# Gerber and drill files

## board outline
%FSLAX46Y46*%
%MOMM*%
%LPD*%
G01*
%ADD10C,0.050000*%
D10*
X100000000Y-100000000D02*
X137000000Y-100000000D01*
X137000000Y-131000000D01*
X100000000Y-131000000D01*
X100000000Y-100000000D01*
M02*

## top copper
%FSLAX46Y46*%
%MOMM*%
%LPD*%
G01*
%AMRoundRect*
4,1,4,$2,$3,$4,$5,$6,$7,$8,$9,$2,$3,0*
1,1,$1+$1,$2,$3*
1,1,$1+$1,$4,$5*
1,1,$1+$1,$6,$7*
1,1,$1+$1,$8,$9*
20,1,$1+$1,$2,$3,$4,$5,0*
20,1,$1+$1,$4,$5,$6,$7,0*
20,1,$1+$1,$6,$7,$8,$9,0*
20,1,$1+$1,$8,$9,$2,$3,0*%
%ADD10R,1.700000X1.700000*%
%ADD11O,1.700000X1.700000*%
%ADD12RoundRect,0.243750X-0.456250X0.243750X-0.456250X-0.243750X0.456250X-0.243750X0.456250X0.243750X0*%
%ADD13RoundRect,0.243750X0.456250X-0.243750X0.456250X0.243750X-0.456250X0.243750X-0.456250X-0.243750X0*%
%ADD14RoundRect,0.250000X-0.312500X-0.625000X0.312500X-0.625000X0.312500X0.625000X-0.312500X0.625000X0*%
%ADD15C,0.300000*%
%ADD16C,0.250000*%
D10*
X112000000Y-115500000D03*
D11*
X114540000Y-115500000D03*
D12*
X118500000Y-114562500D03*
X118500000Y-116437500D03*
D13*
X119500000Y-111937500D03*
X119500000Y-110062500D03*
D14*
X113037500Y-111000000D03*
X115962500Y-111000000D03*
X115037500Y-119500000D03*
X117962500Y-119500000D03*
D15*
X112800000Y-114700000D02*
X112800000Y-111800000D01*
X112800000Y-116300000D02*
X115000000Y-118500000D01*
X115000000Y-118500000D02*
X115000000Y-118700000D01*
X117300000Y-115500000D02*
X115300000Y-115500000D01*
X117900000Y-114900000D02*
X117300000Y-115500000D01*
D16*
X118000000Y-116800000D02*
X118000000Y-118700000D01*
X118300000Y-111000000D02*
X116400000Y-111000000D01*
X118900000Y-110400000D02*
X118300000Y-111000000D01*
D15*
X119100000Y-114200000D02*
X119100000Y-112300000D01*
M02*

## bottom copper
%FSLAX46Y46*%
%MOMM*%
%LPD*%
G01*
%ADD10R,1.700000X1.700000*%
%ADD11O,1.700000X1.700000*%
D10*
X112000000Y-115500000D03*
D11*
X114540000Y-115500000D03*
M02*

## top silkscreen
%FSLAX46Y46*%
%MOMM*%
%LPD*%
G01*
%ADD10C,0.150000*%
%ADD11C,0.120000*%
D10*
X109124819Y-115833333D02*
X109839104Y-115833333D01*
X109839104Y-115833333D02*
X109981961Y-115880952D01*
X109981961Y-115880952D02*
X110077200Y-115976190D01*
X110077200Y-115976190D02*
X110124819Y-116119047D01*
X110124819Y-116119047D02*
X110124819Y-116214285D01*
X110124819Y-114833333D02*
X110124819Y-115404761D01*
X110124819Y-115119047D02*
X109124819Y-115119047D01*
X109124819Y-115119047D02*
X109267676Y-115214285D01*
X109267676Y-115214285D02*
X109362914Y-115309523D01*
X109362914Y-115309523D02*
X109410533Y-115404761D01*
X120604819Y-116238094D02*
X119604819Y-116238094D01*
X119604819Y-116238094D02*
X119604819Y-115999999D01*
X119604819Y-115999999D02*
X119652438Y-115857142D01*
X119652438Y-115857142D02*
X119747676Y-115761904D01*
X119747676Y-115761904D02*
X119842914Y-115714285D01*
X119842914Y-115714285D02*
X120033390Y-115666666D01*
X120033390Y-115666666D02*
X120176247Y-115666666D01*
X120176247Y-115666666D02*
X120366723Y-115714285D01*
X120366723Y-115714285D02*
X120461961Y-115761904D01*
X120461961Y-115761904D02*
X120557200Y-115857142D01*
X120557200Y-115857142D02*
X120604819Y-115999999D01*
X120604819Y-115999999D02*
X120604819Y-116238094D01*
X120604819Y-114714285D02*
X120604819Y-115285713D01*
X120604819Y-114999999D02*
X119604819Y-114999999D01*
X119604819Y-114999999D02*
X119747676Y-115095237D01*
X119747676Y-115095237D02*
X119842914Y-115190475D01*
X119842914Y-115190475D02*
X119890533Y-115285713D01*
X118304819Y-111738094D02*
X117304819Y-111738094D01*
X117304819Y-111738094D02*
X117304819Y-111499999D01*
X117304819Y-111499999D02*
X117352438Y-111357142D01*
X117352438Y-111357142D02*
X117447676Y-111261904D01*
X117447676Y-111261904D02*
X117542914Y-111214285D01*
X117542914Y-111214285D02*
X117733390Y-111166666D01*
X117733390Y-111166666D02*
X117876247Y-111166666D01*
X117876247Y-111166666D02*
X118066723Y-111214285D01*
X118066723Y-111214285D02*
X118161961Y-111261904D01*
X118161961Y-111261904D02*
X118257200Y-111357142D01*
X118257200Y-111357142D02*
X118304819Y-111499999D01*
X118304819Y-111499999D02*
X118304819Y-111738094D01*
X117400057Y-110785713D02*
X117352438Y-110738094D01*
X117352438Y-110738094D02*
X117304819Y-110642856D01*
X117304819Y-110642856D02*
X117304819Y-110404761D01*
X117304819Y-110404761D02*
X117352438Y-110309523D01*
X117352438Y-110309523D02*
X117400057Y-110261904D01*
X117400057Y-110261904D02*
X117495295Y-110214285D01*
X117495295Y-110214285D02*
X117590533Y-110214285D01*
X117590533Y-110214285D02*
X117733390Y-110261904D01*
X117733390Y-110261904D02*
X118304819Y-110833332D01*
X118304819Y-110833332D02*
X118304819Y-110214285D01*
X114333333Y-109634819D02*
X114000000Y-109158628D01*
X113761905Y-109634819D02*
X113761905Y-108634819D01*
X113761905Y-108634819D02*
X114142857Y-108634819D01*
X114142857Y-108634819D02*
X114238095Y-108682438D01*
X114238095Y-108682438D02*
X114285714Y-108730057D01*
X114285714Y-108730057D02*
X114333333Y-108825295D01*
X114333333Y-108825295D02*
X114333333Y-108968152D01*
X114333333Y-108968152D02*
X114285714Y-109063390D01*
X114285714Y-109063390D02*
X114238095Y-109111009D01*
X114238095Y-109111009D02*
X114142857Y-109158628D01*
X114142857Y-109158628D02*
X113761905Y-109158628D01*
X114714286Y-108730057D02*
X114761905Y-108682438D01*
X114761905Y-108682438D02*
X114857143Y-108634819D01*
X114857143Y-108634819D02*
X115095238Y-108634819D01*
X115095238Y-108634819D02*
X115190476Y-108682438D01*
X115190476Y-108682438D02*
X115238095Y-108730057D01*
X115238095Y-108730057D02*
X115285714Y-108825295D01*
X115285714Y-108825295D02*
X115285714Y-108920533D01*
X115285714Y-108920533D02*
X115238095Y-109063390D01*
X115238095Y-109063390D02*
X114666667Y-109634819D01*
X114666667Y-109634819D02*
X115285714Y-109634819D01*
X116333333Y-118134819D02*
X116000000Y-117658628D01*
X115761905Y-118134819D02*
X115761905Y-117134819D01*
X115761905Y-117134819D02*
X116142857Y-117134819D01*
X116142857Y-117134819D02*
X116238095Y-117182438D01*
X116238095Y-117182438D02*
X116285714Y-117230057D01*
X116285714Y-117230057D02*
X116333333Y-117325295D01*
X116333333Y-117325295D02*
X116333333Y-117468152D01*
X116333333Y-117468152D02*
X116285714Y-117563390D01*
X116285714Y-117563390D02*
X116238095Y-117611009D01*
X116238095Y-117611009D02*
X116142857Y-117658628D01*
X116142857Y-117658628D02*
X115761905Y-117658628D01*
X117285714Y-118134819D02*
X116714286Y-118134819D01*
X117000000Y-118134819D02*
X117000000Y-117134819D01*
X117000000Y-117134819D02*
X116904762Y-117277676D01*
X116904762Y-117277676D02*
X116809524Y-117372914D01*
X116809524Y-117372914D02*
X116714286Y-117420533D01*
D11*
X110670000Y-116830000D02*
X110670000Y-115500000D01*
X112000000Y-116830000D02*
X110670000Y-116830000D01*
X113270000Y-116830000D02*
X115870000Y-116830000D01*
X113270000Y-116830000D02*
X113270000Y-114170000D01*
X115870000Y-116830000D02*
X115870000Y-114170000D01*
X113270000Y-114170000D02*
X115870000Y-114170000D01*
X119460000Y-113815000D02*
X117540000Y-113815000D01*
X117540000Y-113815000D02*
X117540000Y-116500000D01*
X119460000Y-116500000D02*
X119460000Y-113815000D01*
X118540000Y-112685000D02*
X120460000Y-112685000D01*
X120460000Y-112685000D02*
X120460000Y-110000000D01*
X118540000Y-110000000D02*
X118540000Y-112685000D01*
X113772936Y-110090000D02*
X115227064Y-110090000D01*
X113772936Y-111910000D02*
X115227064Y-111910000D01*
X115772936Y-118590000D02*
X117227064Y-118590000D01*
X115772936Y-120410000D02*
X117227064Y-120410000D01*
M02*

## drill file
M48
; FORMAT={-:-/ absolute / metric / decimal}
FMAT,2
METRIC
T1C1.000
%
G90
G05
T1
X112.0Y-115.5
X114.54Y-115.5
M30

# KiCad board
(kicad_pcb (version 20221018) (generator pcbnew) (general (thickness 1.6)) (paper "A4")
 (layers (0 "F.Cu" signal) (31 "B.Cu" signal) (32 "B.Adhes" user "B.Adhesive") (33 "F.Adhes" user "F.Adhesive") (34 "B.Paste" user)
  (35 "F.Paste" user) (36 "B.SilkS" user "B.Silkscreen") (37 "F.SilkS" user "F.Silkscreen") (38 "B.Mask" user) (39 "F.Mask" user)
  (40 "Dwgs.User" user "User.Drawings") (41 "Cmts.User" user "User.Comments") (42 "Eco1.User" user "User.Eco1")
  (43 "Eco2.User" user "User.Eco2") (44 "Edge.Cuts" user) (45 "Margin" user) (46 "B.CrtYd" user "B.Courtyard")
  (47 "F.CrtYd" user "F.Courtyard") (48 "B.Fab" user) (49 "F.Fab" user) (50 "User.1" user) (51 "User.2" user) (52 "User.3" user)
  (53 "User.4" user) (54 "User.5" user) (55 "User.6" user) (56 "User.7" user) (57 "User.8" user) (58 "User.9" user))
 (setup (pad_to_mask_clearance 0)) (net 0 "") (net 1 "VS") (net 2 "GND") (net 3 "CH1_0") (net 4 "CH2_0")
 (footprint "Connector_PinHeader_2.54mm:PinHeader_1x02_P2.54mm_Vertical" (layer "F.Cu") (at 112 115.5 90)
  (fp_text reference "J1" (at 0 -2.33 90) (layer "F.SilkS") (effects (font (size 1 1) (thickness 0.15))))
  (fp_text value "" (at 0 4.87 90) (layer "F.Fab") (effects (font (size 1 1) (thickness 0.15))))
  (fp_line (start -1.33 -1.33) (end 0 -1.33) (stroke (width 0.12) (type solid)) (layer "F.SilkS"))
  (fp_line (start -1.33 0) (end -1.33 -1.33) (stroke (width 0.12) (type solid)) (layer "F.SilkS"))
  (fp_line (start -1.33 1.27) (end -1.33 3.87) (stroke (width 0.12) (type solid)) (layer "F.SilkS"))
  (fp_line (start -1.33 1.27) (end 1.33 1.27) (stroke (width 0.12) (type solid)) (layer "F.SilkS"))
  (fp_line (start -1.33 3.87) (end 1.33 3.87) (stroke (width 0.12) (type solid)) (layer "F.SilkS"))
  (fp_line (start 1.33 1.27) (end 1.33 3.87) (stroke (width 0.12) (type solid)) (layer "F.SilkS"))
  (pad "1" thru_hole rect (at 0 0 90) (size 1.7 1.7) (drill 1) (layers "*.Cu" "*.Mask") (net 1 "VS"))
  (pad "2" thru_hole oval (at 0 2.54 90) (size 1.7 1.7) (drill 1) (layers "*.Cu" "*.Mask") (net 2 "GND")))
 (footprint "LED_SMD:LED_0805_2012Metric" (layer "F.Cu") (at 118.5 115.5 -90)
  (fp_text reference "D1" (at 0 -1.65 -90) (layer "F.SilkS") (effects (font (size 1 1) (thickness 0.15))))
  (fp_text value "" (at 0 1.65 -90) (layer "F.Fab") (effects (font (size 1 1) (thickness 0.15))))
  (fp_line (start -1.685 -0.96) (end -1.685 0.96) (stroke (width 0.12) (type solid)) (layer "F.SilkS"))
  (fp_line (start -1.685 0.96) (end 1 0.96) (stroke (width 0.12) (type solid)) (layer "F.SilkS"))
  (fp_line (start 1 -0.96) (end -1.685 -0.96) (stroke (width 0.12) (type solid)) (layer "F.SilkS"))
  (pad "1" smd roundrect (at -0.9375 0 270) (size 0.975 1.4) (layers "F.Cu" "F.Paste" "F.Mask") (roundrect_rratio 0.25) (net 2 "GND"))
  (pad "2" smd roundrect (at 0.9375 0 270) (size 0.975 1.4) (layers "F.Cu" "F.Paste" "F.Mask") (roundrect_rratio 0.25) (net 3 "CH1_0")))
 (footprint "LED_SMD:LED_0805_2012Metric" (layer "F.Cu") (at 119.5 111 90)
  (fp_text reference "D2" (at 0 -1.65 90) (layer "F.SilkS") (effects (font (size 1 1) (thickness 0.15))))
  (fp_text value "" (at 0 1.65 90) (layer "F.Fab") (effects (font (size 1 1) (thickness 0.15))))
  (fp_line (start -1.685 -0.96) (end -1.685 0.96) (stroke (width 0.12) (type solid)) (layer "F.SilkS"))
  (fp_line (start -1.685 0.96) (end 1 0.96) (stroke (width 0.12) (type solid)) (layer "F.SilkS"))
  (fp_line (start 1 -0.96) (end -1.685 -0.96) (stroke (width 0.12) (type solid)) (layer "F.SilkS"))
  (pad "1" smd roundrect (at -0.9375 0 90) (size 0.975 1.4) (layers "F.Cu" "F.Paste" "F.Mask") (roundrect_rratio 0.25) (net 2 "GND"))
  (pad "2" smd roundrect (at 0.9375 0 90) (size 0.975 1.4) (layers "F.Cu" "F.Paste" "F.Mask") (roundrect_rratio 0.25) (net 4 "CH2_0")))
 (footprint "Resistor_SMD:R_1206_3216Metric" (layer "F.Cu") (at 114.5 111)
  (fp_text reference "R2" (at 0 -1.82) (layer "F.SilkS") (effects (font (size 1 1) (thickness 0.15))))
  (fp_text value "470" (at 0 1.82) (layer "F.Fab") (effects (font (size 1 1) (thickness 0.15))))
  (fp_line (start -0.727064 -0.91) (end 0.727064 -0.91) (stroke (width 0.12) (type solid)) (layer "F.SilkS"))
  (fp_line (start -0.727064 0.91) (end 0.727064 0.91) (stroke (width 0.12) (type solid)) (layer "F.SilkS"))
  (pad "1" smd roundrect (at -1.4625 0) (size 1.125 1.75) (layers "F.Cu" "F.Paste" "F.Mask") (roundrect_rratio 0.222222) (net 1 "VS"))
  (pad "2" smd roundrect (at 1.4625 0) (size 1.125 1.75) (layers "F.Cu" "F.Paste" "F.Mask") (roundrect_rratio 0.222222) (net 4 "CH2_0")))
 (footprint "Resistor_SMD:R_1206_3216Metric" (layer "F.Cu") (at 116.5 119.5)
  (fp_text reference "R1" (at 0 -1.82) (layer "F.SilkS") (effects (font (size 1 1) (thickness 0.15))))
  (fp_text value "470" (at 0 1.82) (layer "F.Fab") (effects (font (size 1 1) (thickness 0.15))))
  (fp_line (start -0.727064 -0.91) (end 0.727064 -0.91) (stroke (width 0.12) (type solid)) (layer "F.SilkS"))
  (fp_line (start -0.727064 0.91) (end 0.727064 0.91) (stroke (width 0.12) (type solid)) (layer "F.SilkS"))
  (pad "1" smd roundrect (at -1.4625 0) (size 1.125 1.75) (layers "F.Cu" "F.Paste" "F.Mask") (roundrect_rratio 0.222222) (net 1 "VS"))
  (pad "2" smd roundrect (at 1.4625 0) (size 1.125 1.75) (layers "F.Cu" "F.Paste" "F.Mask") (roundrect_rratio 0.222222) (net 3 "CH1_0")))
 (gr_rect (start 100 100) (end 137 131) (stroke (width 0.05) (type default)) (fill none) (layer "Edge.Cuts"))
 (segment (start 112.8 114.7) (end 112.8 111.8) (width 0.3) (layer "F.Cu") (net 1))
 (segment (start 112.8 116.3) (end 115 118.5) (width 0.3) (layer "F.Cu") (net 1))
 (segment (start 115 118.5) (end 115 118.7) (width 0.3) (layer "F.Cu") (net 1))
 (segment (start 117.3 115.5) (end 115.3 115.5) (width 0.3) (layer "F.Cu") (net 2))
 (segment (start 117.9 114.9) (end 117.3 115.5) (width 0.3) (layer "F.Cu") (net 2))
 (segment (start 118 116.8) (end 118 118.7) (width 0.25) (layer "F.Cu") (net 3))
 (segment (start 118.3 111) (end 116.4 111) (width 0.25) (layer "F.Cu") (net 4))
 (segment (start 118.9 110.4) (end 118.3 111) (width 0.25) (layer "F.Cu") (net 4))
 (segment (start 119.1 114.2) (end 119.1 112.3) (width 0.3) (layer "F.Cu") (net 2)))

